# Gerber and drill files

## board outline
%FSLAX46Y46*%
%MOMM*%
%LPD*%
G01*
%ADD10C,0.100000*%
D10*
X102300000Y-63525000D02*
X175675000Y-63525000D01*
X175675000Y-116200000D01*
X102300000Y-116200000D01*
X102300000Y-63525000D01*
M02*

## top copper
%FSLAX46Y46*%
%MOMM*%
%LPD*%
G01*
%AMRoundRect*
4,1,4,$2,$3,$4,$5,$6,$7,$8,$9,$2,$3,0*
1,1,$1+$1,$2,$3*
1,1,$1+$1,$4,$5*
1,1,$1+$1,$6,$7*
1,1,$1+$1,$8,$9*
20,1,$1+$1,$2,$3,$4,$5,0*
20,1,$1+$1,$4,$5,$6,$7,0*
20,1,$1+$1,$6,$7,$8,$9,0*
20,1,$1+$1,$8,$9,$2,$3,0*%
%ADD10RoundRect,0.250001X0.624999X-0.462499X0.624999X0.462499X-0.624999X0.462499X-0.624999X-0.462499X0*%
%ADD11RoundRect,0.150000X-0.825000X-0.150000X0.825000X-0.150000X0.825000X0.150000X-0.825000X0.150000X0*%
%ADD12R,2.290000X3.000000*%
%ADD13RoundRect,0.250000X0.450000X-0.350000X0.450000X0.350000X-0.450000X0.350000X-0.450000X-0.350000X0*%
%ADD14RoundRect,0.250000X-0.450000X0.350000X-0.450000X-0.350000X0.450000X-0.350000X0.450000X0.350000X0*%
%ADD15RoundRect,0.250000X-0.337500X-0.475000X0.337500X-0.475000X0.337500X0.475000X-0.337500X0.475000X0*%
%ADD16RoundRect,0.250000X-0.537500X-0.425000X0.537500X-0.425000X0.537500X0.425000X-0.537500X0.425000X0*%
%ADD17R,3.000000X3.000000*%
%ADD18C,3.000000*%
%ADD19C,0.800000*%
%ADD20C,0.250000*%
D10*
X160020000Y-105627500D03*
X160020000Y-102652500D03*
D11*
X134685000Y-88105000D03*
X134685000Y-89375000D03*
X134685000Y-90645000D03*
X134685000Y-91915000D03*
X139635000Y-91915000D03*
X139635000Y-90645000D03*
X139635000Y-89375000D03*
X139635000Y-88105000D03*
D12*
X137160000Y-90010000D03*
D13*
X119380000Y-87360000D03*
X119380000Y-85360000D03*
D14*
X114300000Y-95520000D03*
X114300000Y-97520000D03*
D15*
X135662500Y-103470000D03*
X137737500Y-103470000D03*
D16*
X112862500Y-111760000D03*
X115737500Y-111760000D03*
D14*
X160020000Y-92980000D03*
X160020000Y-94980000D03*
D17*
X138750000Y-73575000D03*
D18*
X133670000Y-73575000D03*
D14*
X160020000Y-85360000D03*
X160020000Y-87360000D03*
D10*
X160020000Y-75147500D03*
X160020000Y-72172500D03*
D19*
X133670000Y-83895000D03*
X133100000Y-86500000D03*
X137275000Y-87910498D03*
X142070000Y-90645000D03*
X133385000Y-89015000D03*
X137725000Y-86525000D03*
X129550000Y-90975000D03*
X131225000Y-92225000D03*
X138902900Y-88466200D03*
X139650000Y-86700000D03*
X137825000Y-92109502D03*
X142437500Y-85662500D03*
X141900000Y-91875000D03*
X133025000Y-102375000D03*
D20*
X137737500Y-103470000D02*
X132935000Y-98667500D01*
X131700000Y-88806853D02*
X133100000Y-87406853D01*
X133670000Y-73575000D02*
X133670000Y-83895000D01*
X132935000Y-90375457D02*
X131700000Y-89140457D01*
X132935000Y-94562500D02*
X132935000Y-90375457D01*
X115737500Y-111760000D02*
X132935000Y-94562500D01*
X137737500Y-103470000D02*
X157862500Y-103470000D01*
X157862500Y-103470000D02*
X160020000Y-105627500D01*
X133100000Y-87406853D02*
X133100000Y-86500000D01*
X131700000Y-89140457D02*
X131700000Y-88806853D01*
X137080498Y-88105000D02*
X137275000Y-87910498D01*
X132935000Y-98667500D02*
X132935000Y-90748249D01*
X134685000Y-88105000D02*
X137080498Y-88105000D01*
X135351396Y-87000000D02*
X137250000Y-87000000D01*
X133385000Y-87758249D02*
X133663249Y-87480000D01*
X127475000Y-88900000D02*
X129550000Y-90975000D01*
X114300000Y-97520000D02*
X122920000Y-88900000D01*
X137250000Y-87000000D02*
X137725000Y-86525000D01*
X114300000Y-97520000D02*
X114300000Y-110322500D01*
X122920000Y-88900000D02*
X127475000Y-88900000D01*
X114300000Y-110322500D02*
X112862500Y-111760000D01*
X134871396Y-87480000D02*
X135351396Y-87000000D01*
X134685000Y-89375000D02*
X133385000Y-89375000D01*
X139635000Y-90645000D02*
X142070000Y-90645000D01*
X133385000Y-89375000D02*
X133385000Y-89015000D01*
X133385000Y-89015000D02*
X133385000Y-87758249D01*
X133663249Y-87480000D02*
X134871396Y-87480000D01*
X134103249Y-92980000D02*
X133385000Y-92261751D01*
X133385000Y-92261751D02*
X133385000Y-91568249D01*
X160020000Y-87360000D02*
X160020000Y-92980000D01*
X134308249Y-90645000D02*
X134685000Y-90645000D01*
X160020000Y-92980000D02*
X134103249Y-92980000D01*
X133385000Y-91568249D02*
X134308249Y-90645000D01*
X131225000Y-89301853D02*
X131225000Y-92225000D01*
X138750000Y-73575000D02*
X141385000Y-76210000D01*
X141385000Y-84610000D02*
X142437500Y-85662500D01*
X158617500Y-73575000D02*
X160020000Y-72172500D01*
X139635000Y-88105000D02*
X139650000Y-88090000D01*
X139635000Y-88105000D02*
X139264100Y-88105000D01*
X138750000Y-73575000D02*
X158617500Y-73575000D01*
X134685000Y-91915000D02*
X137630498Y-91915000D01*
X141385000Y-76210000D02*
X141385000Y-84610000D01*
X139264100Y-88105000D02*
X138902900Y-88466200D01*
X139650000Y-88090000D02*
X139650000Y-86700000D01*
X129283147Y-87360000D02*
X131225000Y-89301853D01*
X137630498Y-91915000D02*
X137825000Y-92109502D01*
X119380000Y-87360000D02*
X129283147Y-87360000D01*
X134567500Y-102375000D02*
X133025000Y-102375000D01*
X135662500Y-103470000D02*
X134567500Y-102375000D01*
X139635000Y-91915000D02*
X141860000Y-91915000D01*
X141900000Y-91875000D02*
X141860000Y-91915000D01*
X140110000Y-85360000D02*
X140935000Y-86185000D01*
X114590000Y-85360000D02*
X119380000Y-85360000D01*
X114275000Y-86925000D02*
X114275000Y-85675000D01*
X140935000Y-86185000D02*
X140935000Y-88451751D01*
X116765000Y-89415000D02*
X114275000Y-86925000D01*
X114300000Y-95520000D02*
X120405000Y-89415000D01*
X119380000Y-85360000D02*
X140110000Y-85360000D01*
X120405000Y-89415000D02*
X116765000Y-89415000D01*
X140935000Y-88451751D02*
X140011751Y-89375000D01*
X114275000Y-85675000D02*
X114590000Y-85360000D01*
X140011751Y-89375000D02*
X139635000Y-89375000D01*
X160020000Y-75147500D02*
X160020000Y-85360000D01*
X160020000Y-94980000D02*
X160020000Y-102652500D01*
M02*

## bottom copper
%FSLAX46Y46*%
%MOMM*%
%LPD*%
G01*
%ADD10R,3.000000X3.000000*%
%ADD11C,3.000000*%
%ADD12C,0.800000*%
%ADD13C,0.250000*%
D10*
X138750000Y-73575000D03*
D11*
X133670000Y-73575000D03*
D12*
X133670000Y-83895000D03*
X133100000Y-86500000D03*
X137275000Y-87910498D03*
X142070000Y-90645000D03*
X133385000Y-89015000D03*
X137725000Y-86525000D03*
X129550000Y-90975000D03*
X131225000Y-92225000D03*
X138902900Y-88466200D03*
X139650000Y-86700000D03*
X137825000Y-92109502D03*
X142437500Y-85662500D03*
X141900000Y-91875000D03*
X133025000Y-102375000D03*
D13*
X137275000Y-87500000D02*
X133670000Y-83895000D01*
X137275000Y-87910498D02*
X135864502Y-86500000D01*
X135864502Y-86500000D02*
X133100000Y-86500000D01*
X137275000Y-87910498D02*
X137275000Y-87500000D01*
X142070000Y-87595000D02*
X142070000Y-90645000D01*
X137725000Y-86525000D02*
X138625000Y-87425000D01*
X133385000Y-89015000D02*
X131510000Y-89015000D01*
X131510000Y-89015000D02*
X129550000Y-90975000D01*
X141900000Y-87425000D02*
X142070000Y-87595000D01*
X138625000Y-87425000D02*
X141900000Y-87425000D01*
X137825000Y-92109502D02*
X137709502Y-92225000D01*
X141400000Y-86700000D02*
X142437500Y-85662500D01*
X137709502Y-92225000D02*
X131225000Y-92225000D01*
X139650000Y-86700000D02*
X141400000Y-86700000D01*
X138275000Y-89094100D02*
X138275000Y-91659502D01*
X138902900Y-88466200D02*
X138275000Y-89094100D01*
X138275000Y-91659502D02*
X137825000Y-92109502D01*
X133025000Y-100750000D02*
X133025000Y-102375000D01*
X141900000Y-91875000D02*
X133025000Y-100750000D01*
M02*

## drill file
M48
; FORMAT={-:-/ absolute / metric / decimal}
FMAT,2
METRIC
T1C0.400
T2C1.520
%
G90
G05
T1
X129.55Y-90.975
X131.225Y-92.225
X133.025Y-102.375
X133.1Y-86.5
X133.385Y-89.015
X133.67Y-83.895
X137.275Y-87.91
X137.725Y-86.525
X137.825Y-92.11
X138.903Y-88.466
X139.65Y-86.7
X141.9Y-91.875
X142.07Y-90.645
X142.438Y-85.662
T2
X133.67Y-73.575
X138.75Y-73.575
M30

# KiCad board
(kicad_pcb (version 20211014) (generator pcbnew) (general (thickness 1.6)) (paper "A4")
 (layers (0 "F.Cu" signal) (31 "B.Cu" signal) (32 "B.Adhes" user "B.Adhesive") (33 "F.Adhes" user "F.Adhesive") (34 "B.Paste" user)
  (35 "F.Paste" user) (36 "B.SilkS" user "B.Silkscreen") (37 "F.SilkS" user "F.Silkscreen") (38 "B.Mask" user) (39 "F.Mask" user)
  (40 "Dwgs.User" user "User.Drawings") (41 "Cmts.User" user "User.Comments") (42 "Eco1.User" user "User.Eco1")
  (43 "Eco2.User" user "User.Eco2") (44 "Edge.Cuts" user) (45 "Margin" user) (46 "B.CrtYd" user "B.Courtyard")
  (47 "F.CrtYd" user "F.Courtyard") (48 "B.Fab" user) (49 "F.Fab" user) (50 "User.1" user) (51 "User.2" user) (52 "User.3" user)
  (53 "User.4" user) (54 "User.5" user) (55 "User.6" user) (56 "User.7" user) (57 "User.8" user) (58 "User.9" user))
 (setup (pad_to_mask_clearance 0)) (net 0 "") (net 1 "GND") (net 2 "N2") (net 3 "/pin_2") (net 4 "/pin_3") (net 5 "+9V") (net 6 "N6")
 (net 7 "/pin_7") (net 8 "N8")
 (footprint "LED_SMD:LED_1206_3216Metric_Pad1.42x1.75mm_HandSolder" (layer "F.Cu") (at 160.02 104.14 90)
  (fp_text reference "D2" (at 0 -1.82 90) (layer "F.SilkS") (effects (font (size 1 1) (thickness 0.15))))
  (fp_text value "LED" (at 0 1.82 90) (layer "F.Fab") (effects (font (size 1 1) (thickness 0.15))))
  (pad "1" smd roundrect (at -1.4875 0 90) (size 1.425 1.75) (layers "F.Cu" "F.Paste" "F.Mask") (roundrect_rratio 0.1754392982)
   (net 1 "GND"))
  (pad "2" smd roundrect (at 1.4875 0 90) (size 1.425 1.75) (layers "F.Cu" "F.Paste" "F.Mask") (roundrect_rratio 0.1754392982) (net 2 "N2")))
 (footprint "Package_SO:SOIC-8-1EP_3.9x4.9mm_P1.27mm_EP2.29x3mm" (layer "F.Cu") (at 137.16 90.01)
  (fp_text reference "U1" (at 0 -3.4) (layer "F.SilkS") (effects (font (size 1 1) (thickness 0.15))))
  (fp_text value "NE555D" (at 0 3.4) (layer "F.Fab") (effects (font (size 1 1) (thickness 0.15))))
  (pad "" smd roundrect (at 0.57 -0.75) (size 0.92 1.21) (layers "F.Paste") (roundrect_rratio 0.25))
  (pad "" smd roundrect (at 0.57 0.75) (size 0.92 1.21) (layers "F.Paste") (roundrect_rratio 0.25))
  (pad "" smd roundrect (at -0.57 -0.75) (size 0.92 1.21) (layers "F.Paste") (roundrect_rratio 0.25))
  (pad "" smd roundrect (at -0.57 0.75) (size 0.92 1.21) (layers "F.Paste") (roundrect_rratio 0.25))
  (pad "1" smd roundrect (at -2.475 -1.905) (size 1.95 0.6) (layers "F.Cu" "F.Paste" "F.Mask") (roundrect_rratio 0.25) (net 1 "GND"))
  (pad "2" smd roundrect (at -2.475 -0.635) (size 1.95 0.6) (layers "F.Cu" "F.Paste" "F.Mask") (roundrect_rratio 0.25) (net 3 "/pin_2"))
  (pad "3" smd roundrect (at -2.475 0.635) (size 1.95 0.6) (layers "F.Cu" "F.Paste" "F.Mask") (roundrect_rratio 0.25) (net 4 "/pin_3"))
  (pad "4" smd roundrect (at -2.475 1.905) (size 1.95 0.6) (layers "F.Cu" "F.Paste" "F.Mask") (roundrect_rratio 0.25) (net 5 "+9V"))
  (pad "5" smd roundrect (at 2.475 1.905) (size 1.95 0.6) (layers "F.Cu" "F.Paste" "F.Mask") (roundrect_rratio 0.25) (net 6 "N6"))
  (pad "6" smd roundrect (at 2.475 0.635) (size 1.95 0.6) (layers "F.Cu" "F.Paste" "F.Mask") (roundrect_rratio 0.25) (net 3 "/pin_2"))
  (pad "7" smd roundrect (at 2.475 -0.635) (size 1.95 0.6) (layers "F.Cu" "F.Paste" "F.Mask") (roundrect_rratio 0.25) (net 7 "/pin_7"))
  (pad "8" smd roundrect (at 2.475 -1.905) (size 1.95 0.6) (layers "F.Cu" "F.Paste" "F.Mask") (roundrect_rratio 0.25) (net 5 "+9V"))
  (pad "9" smd rect (at 0 0) (size 2.29 3) (layers "F.Cu" "F.Mask")))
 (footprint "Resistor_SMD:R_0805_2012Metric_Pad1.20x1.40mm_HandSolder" (layer "F.Cu") (at 119.38 86.36 90)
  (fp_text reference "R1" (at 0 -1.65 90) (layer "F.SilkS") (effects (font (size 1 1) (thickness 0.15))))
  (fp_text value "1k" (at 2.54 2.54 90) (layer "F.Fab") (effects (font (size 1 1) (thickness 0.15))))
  (pad "1" smd roundrect (at -1 0 90) (size 1.2 1.4) (layers "F.Cu" "F.Paste" "F.Mask") (roundrect_rratio 0.2083333333) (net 5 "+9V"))
  (pad "2" smd roundrect (at 1 0 90) (size 1.2 1.4) (layers "F.Cu" "F.Paste" "F.Mask") (roundrect_rratio 0.2083333333) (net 7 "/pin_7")))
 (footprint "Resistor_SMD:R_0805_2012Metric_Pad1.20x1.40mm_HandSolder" (layer "F.Cu") (at 114.3 96.52 -90)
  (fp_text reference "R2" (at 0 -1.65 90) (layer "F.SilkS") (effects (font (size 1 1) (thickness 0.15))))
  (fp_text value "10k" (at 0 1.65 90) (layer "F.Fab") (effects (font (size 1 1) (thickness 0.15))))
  (pad "1" smd roundrect (at -1 0 270) (size 1.2 1.4) (layers "F.Cu" "F.Paste" "F.Mask") (roundrect_rratio 0.2083333333) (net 7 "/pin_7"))
  (pad "2" smd roundrect (at 1 0 270) (size 1.2 1.4) (layers "F.Cu" "F.Paste" "F.Mask") (roundrect_rratio 0.2083333333) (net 3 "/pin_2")))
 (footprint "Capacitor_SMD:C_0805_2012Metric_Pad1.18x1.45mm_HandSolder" (layer "F.Cu") (at 136.7 103.47)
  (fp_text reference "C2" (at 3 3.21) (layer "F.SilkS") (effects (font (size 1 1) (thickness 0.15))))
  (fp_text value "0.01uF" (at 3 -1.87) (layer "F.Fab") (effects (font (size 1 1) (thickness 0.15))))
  (pad "1" smd roundrect (at -1.0375 0) (size 1.175 1.45) (layers "F.Cu" "F.Paste" "F.Mask") (roundrect_rratio 0.2127659574) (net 6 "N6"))
  (pad "2" smd roundrect (at 1.0375 0) (size 1.175 1.45) (layers "F.Cu" "F.Paste" "F.Mask") (roundrect_rratio 0.2127659574) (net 1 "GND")))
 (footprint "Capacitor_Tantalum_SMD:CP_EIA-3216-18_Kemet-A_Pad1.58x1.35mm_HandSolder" (layer "F.Cu") (at 114.3 111.76)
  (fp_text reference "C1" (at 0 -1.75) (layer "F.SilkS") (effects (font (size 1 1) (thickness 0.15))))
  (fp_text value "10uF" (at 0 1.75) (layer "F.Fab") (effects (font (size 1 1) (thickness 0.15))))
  (pad "1" smd roundrect (at -1.4375 0) (size 1.575 1.35) (layers "F.Cu" "F.Paste" "F.Mask") (roundrect_rratio 0.1851851852)
   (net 3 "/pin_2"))
  (pad "2" smd roundrect (at 1.4375 0) (size 1.575 1.35) (layers "F.Cu" "F.Paste" "F.Mask") (roundrect_rratio 0.1851851852) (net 1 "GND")))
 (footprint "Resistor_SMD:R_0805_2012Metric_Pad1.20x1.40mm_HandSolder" (layer "F.Cu") (at 160.02 93.98 -90)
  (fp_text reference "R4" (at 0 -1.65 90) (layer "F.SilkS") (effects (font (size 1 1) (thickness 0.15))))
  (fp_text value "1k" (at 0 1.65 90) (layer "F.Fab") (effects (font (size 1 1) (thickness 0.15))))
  (pad "1" smd roundrect (at -1 0 270) (size 1.2 1.4) (layers "F.Cu" "F.Paste" "F.Mask") (roundrect_rratio 0.2083333333) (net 4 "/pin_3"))
  (pad "2" smd roundrect (at 1 0 270) (size 1.2 1.4) (layers "F.Cu" "F.Paste" "F.Mask") (roundrect_rratio 0.2083333333) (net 2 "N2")))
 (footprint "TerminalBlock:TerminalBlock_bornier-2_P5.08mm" (layer "F.Cu") (at 138.75 73.575 180)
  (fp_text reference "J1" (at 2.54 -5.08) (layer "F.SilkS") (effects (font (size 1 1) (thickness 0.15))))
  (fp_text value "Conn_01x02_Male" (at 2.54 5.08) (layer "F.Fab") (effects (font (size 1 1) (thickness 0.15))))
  (pad "1" thru_hole rect (at 0 0 180) (size 3 3) (drill 1.52) (layers *.Cu *.Mask) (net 5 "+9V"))
  (pad "2" thru_hole circle (at 5.08 0 180) (size 3 3) (drill 1.52) (layers *.Cu *.Mask) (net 1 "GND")))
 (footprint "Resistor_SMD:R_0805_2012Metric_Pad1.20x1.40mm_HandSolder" (layer "F.Cu") (at 160.02 86.36 -90)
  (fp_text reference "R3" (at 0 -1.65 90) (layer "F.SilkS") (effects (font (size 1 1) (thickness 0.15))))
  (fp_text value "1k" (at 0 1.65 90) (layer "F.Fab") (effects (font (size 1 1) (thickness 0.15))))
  (pad "1" smd roundrect (at -1 0 270) (size 1.2 1.4) (layers "F.Cu" "F.Paste" "F.Mask") (roundrect_rratio 0.2083333333) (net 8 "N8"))
  (pad "2" smd roundrect (at 1 0 270) (size 1.2 1.4) (layers "F.Cu" "F.Paste" "F.Mask") (roundrect_rratio 0.2083333333) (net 4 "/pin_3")))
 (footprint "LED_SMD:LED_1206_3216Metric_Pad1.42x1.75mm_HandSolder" (layer "F.Cu") (at 160.02 73.66 90)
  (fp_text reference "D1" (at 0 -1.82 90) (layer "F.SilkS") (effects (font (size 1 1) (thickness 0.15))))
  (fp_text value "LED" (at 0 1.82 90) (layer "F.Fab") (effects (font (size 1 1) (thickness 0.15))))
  (pad "1" smd roundrect (at -1.4875 0 90) (size 1.425 1.75) (layers "F.Cu" "F.Paste" "F.Mask") (roundrect_rratio 0.1754392982) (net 8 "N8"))
  (pad "2" smd roundrect (at 1.4875 0 90) (size 1.425 1.75) (layers "F.Cu" "F.Paste" "F.Mask") (roundrect_rratio 0.1754392982) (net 5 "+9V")))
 (gr_rect (start 175.675 63.525) (end 102.3 116.2) (layer "Edge.Cuts") (width 0.1) (fill none))
 (segment (start 137.7375 103.47) (end 132.935 98.6675) (width 0.25) (layer "F.Cu") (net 1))
 (segment (start 131.7 88.806853) (end 133.1 87.406853) (width 0.25) (layer "F.Cu") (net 1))
 (segment (start 133.67 73.575) (end 133.67 83.895) (width 0.25) (layer "F.Cu") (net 1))
 (segment (start 132.935 90.375457) (end 131.7 89.140457) (width 0.25) (layer "F.Cu") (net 1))
 (segment (start 132.935 94.5625) (end 132.935 90.375457) (width 0.25) (layer "F.Cu") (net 1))
 (segment (start 115.7375 111.76) (end 132.935 94.5625) (width 0.25) (layer "F.Cu") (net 1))
 (segment (start 137.7375 103.47) (end 157.8625 103.47) (width 0.25) (layer "F.Cu") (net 1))
 (segment (start 157.8625 103.47) (end 160.02 105.6275) (width 0.25) (layer "F.Cu") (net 1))
 (segment (start 133.1 87.406853) (end 133.1 86.5) (width 0.25) (layer "F.Cu") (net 1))
 (segment (start 131.7 89.140457) (end 131.7 88.806853) (width 0.25) (layer "F.Cu") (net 1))
 (segment (start 137.080498 88.105) (end 137.275 87.910498) (width 0.25) (layer "F.Cu") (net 1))
 (segment (start 132.935 98.6675) (end 132.935 90.748249) (width 0.25) (layer "F.Cu") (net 1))
 (segment (start 134.685 88.105) (end 137.080498 88.105) (width 0.25) (layer "F.Cu") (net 1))
 (via (at 133.67 83.895) (size 0.8) (drill 0.4) (layers "F.Cu" "B.Cu") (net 1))
 (via (at 133.1 86.5) (size 0.8) (drill 0.4) (layers "F.Cu" "B.Cu") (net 1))
 (via (at 137.275 87.910498) (size 0.8) (drill 0.4) (layers "F.Cu" "B.Cu") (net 1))
 (segment (start 137.275 87.5) (end 133.67 83.895) (width 0.25) (layer "B.Cu") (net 1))
 (segment (start 137.275 87.910498) (end 135.864502 86.5) (width 0.25) (layer "B.Cu") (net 1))
 (segment (start 135.864502 86.5) (end 133.1 86.5) (width 0.25) (layer "B.Cu") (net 1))
 (segment (start 137.275 87.910498) (end 137.275 87.5) (width 0.25) (layer "B.Cu") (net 1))
 (segment (start 135.351396 87) (end 137.25 87) (width 0.25) (layer "F.Cu") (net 3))
 (segment (start 133.385 87.758249) (end 133.663249 87.48) (width 0.25) (layer "F.Cu") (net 3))
 (segment (start 127.475 88.9) (end 129.55 90.975) (width 0.25) (layer "F.Cu") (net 3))
 (segment (start 114.3 97.52) (end 122.92 88.9) (width 0.25) (layer "F.Cu") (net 3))
 (segment (start 137.25 87) (end 137.725 86.525) (width 0.25) (layer "F.Cu") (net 3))
 (segment (start 114.3 97.52) (end 114.3 110.3225) (width 0.25) (layer "F.Cu") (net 3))
 (segment (start 122.92 88.9) (end 127.475 88.9) (width 0.25) (layer "F.Cu") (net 3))
 (segment (start 114.3 110.3225) (end 112.8625 111.76) (width 0.25) (layer "F.Cu") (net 3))
 (segment (start 134.871396 87.48) (end 135.351396 87) (width 0.25) (layer "F.Cu") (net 3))
 (segment (start 134.685 89.375) (end 133.385 89.375) (width 0.25) (layer "F.Cu") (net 3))
 (segment (start 139.635 90.645) (end 142.07 90.645) (width 0.25) (layer "F.Cu") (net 3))
 (segment (start 133.385 89.375) (end 133.385 89.015) (width 0.25) (layer "F.Cu") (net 3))
 (segment (start 133.385 89.015) (end 133.385 87.758249) (width 0.25) (layer "F.Cu") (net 3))
 (segment (start 133.663249 87.48) (end 134.871396 87.48) (width 0.25) (layer "F.Cu") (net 3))
 (via (at 142.07 90.645) (size 0.8) (drill 0.4) (layers "F.Cu" "B.Cu") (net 3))
 (via (at 133.385 89.015) (size 0.8) (drill 0.4) (layers "F.Cu" "B.Cu") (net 3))
 (via (at 137.725 86.525) (size 0.8) (drill 0.4) (layers "F.Cu" "B.Cu") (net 3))
 (via (at 129.55 90.975) (size 0.8) (drill 0.4) (layers "F.Cu" "B.Cu") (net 3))
 (segment (start 142.07 87.595) (end 142.07 90.645) (width 0.25) (layer "B.Cu") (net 3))
 (segment (start 137.725 86.525) (end 138.625 87.425) (width 0.25) (layer "B.Cu") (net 3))
 (segment (start 133.385 89.015) (end 131.51 89.015) (width 0.25) (layer "B.Cu") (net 3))
 (segment (start 131.51 89.015) (end 129.55 90.975) (width 0.25) (layer "B.Cu") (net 3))
 (segment (start 141.9 87.425) (end 142.07 87.595) (width 0.25) (layer "B.Cu") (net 3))
 (segment (start 138.625 87.425) (end 141.9 87.425) (width 0.25) (layer "B.Cu") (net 3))
 (segment (start 134.103249 92.98) (end 133.385 92.261751) (width 0.25) (layer "F.Cu") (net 4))
 (segment (start 133.385 92.261751) (end 133.385 91.568249) (width 0.25) (layer "F.Cu") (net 4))
 (segment (start 160.02 87.36) (end 160.02 92.98) (width 0.25) (layer "F.Cu") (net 4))
 (segment (start 134.308249 90.645) (end 134.685 90.645) (width 0.25) (layer "F.Cu") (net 4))
 (segment (start 160.02 92.98) (end 134.103249 92.98) (width 0.25) (layer "F.Cu") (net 4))
 (segment (start 133.385 91.568249) (end 134.308249 90.645) (width 0.25) (layer "F.Cu") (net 4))
 (segment (start 131.225 89.301853) (end 131.225 92.225) (width 0.25) (layer "F.Cu") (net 5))
 (segment (start 138.75 73.575) (end 141.385 76.21) (width 0.25) (layer "F.Cu") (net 5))
 (segment (start 141.385 84.61) (end 142.4375 85.6625) (width 0.25) (layer "F.Cu") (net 5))
 (segment (start 158.6175 73.575) (end 160.02 72.1725) (width 0.25) (layer "F.Cu") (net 5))
 (segment (start 139.635 88.105) (end 139.65 88.09) (width 0.25) (layer "F.Cu") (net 5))
 (segment (start 139.635 88.105) (end 139.2641 88.105) (width 0.25) (layer "F.Cu") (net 5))
 (segment (start 138.75 73.575) (end 158.6175 73.575) (width 0.25) (layer "F.Cu") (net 5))
 (segment (start 134.685 91.915) (end 137.630498 91.915) (width 0.25) (layer "F.Cu") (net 5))
 (segment (start 141.385 76.21) (end 141.385 84.61) (width 0.25) (layer "F.Cu") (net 5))
 (segment (start 139.2641 88.105) (end 138.9029 88.4662) (width 0.25) (layer "F.Cu") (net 5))
 (segment (start 139.65 88.09) (end 139.65 86.7) (width 0.25) (layer "F.Cu") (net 5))
 (segment (start 129.283147 87.36) (end 131.225 89.301853) (width 0.25) (layer "F.Cu") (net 5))
 (segment (start 137.630498 91.915) (end 137.825 92.109502) (width 0.25) (layer "F.Cu") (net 5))
 (segment (start 119.38 87.36) (end 129.283147 87.36) (width 0.25) (layer "F.Cu") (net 5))
 (via (at 131.225 92.225) (size 0.8) (drill 0.4) (layers "F.Cu" "B.Cu") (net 5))
 (via (at 138.9029 88.4662) (size 0.8) (drill 0.4) (layers "F.Cu" "B.Cu") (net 5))
 (via (at 139.65 86.7) (size 0.8) (drill 0.4) (layers "F.Cu" "B.Cu") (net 5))
 (via (at 137.825 92.109502) (size 0.8) (drill 0.4) (layers "F.Cu" "B.Cu") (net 5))
 (via (at 142.4375 85.6625) (size 0.8) (drill 0.4) (layers "F.Cu" "B.Cu") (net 5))
 (segment (start 137.825 92.109502) (end 137.709502 92.225) (width 0.25) (layer "B.Cu") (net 5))
 (segment (start 141.4 86.7) (end 142.4375 85.6625) (width 0.25) (layer "B.Cu") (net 5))
 (segment (start 137.709502 92.225) (end 131.225 92.225) (width 0.25) (layer "B.Cu") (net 5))
 (segment (start 139.65 86.7) (end 141.4 86.7) (width 0.25) (layer "B.Cu") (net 5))
 (segment (start 138.275 89.0941) (end 138.275 91.659502) (width 0.25) (layer "B.Cu") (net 5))
 (segment (start 138.9029 88.4662) (end 138.275 89.0941) (width 0.25) (layer "B.Cu") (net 5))
 (segment (start 138.275 91.659502) (end 137.825 92.109502) (width 0.25) (layer "B.Cu") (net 5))
 (segment (start 134.5675 102.375) (end 133.025 102.375) (width 0.25) (layer "F.Cu") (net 6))
 (segment (start 135.6625 103.47) (end 134.5675 102.375) (width 0.25) (layer "F.Cu") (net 6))
 (segment (start 139.635 91.915) (end 141.86 91.915) (width 0.25) (layer "F.Cu") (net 6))
 (segment (start 141.9 91.875) (end 141.86 91.915) (width 0.25) (layer "F.Cu") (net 6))
 (via (at 141.9 91.875) (size 0.8) (drill 0.4) (layers "F.Cu" "B.Cu") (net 6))
 (via (at 133.025 102.375) (size 0.8) (drill 0.4) (layers "F.Cu" "B.Cu") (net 6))
 (segment (start 133.025 100.75) (end 133.025 102.375) (width 0.25) (layer "B.Cu") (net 6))
 (segment (start 141.9 91.875) (end 133.025 100.75) (width 0.25) (layer "B.Cu") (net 6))
 (segment (start 140.11 85.36) (end 140.935 86.185) (width 0.25) (layer "F.Cu") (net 7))
 (segment (start 114.59 85.36) (end 119.38 85.36) (width 0.25) (layer "F.Cu") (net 7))
 (segment (start 114.275 86.925) (end 114.275 85.675) (width 0.25) (layer "F.Cu") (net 7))
 (segment (start 140.935 86.185) (end 140.935 88.451751) (width 0.25) (layer "F.Cu") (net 7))
 (segment (start 116.765 89.415) (end 114.275 86.925) (width 0.25) (layer "F.Cu") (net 7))
 (segment (start 114.3 95.52) (end 120.405 89.415) (width 0.25) (layer "F.Cu") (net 7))
 (segment (start 119.38 85.36) (end 140.11 85.36) (width 0.25) (layer "F.Cu") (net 7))
 (segment (start 120.405 89.415) (end 116.765 89.415) (width 0.25) (layer "F.Cu") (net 7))
 (segment (start 140.935 88.451751) (end 140.011751 89.375) (width 0.25) (layer "F.Cu") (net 7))
 (segment (start 114.275 85.675) (end 114.59 85.36) (width 0.25) (layer "F.Cu") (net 7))
 (segment (start 140.011751 89.375) (end 139.635 89.375) (width 0.25) (layer "F.Cu") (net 7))
 (segment (start 160.02 75.1475) (end 160.02 85.36) (width 0.25) (layer "F.Cu") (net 8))
 (segment (start 160.02 94.98) (end 160.02 102.6525) (width 0.25) (layer "F.Cu") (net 2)))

